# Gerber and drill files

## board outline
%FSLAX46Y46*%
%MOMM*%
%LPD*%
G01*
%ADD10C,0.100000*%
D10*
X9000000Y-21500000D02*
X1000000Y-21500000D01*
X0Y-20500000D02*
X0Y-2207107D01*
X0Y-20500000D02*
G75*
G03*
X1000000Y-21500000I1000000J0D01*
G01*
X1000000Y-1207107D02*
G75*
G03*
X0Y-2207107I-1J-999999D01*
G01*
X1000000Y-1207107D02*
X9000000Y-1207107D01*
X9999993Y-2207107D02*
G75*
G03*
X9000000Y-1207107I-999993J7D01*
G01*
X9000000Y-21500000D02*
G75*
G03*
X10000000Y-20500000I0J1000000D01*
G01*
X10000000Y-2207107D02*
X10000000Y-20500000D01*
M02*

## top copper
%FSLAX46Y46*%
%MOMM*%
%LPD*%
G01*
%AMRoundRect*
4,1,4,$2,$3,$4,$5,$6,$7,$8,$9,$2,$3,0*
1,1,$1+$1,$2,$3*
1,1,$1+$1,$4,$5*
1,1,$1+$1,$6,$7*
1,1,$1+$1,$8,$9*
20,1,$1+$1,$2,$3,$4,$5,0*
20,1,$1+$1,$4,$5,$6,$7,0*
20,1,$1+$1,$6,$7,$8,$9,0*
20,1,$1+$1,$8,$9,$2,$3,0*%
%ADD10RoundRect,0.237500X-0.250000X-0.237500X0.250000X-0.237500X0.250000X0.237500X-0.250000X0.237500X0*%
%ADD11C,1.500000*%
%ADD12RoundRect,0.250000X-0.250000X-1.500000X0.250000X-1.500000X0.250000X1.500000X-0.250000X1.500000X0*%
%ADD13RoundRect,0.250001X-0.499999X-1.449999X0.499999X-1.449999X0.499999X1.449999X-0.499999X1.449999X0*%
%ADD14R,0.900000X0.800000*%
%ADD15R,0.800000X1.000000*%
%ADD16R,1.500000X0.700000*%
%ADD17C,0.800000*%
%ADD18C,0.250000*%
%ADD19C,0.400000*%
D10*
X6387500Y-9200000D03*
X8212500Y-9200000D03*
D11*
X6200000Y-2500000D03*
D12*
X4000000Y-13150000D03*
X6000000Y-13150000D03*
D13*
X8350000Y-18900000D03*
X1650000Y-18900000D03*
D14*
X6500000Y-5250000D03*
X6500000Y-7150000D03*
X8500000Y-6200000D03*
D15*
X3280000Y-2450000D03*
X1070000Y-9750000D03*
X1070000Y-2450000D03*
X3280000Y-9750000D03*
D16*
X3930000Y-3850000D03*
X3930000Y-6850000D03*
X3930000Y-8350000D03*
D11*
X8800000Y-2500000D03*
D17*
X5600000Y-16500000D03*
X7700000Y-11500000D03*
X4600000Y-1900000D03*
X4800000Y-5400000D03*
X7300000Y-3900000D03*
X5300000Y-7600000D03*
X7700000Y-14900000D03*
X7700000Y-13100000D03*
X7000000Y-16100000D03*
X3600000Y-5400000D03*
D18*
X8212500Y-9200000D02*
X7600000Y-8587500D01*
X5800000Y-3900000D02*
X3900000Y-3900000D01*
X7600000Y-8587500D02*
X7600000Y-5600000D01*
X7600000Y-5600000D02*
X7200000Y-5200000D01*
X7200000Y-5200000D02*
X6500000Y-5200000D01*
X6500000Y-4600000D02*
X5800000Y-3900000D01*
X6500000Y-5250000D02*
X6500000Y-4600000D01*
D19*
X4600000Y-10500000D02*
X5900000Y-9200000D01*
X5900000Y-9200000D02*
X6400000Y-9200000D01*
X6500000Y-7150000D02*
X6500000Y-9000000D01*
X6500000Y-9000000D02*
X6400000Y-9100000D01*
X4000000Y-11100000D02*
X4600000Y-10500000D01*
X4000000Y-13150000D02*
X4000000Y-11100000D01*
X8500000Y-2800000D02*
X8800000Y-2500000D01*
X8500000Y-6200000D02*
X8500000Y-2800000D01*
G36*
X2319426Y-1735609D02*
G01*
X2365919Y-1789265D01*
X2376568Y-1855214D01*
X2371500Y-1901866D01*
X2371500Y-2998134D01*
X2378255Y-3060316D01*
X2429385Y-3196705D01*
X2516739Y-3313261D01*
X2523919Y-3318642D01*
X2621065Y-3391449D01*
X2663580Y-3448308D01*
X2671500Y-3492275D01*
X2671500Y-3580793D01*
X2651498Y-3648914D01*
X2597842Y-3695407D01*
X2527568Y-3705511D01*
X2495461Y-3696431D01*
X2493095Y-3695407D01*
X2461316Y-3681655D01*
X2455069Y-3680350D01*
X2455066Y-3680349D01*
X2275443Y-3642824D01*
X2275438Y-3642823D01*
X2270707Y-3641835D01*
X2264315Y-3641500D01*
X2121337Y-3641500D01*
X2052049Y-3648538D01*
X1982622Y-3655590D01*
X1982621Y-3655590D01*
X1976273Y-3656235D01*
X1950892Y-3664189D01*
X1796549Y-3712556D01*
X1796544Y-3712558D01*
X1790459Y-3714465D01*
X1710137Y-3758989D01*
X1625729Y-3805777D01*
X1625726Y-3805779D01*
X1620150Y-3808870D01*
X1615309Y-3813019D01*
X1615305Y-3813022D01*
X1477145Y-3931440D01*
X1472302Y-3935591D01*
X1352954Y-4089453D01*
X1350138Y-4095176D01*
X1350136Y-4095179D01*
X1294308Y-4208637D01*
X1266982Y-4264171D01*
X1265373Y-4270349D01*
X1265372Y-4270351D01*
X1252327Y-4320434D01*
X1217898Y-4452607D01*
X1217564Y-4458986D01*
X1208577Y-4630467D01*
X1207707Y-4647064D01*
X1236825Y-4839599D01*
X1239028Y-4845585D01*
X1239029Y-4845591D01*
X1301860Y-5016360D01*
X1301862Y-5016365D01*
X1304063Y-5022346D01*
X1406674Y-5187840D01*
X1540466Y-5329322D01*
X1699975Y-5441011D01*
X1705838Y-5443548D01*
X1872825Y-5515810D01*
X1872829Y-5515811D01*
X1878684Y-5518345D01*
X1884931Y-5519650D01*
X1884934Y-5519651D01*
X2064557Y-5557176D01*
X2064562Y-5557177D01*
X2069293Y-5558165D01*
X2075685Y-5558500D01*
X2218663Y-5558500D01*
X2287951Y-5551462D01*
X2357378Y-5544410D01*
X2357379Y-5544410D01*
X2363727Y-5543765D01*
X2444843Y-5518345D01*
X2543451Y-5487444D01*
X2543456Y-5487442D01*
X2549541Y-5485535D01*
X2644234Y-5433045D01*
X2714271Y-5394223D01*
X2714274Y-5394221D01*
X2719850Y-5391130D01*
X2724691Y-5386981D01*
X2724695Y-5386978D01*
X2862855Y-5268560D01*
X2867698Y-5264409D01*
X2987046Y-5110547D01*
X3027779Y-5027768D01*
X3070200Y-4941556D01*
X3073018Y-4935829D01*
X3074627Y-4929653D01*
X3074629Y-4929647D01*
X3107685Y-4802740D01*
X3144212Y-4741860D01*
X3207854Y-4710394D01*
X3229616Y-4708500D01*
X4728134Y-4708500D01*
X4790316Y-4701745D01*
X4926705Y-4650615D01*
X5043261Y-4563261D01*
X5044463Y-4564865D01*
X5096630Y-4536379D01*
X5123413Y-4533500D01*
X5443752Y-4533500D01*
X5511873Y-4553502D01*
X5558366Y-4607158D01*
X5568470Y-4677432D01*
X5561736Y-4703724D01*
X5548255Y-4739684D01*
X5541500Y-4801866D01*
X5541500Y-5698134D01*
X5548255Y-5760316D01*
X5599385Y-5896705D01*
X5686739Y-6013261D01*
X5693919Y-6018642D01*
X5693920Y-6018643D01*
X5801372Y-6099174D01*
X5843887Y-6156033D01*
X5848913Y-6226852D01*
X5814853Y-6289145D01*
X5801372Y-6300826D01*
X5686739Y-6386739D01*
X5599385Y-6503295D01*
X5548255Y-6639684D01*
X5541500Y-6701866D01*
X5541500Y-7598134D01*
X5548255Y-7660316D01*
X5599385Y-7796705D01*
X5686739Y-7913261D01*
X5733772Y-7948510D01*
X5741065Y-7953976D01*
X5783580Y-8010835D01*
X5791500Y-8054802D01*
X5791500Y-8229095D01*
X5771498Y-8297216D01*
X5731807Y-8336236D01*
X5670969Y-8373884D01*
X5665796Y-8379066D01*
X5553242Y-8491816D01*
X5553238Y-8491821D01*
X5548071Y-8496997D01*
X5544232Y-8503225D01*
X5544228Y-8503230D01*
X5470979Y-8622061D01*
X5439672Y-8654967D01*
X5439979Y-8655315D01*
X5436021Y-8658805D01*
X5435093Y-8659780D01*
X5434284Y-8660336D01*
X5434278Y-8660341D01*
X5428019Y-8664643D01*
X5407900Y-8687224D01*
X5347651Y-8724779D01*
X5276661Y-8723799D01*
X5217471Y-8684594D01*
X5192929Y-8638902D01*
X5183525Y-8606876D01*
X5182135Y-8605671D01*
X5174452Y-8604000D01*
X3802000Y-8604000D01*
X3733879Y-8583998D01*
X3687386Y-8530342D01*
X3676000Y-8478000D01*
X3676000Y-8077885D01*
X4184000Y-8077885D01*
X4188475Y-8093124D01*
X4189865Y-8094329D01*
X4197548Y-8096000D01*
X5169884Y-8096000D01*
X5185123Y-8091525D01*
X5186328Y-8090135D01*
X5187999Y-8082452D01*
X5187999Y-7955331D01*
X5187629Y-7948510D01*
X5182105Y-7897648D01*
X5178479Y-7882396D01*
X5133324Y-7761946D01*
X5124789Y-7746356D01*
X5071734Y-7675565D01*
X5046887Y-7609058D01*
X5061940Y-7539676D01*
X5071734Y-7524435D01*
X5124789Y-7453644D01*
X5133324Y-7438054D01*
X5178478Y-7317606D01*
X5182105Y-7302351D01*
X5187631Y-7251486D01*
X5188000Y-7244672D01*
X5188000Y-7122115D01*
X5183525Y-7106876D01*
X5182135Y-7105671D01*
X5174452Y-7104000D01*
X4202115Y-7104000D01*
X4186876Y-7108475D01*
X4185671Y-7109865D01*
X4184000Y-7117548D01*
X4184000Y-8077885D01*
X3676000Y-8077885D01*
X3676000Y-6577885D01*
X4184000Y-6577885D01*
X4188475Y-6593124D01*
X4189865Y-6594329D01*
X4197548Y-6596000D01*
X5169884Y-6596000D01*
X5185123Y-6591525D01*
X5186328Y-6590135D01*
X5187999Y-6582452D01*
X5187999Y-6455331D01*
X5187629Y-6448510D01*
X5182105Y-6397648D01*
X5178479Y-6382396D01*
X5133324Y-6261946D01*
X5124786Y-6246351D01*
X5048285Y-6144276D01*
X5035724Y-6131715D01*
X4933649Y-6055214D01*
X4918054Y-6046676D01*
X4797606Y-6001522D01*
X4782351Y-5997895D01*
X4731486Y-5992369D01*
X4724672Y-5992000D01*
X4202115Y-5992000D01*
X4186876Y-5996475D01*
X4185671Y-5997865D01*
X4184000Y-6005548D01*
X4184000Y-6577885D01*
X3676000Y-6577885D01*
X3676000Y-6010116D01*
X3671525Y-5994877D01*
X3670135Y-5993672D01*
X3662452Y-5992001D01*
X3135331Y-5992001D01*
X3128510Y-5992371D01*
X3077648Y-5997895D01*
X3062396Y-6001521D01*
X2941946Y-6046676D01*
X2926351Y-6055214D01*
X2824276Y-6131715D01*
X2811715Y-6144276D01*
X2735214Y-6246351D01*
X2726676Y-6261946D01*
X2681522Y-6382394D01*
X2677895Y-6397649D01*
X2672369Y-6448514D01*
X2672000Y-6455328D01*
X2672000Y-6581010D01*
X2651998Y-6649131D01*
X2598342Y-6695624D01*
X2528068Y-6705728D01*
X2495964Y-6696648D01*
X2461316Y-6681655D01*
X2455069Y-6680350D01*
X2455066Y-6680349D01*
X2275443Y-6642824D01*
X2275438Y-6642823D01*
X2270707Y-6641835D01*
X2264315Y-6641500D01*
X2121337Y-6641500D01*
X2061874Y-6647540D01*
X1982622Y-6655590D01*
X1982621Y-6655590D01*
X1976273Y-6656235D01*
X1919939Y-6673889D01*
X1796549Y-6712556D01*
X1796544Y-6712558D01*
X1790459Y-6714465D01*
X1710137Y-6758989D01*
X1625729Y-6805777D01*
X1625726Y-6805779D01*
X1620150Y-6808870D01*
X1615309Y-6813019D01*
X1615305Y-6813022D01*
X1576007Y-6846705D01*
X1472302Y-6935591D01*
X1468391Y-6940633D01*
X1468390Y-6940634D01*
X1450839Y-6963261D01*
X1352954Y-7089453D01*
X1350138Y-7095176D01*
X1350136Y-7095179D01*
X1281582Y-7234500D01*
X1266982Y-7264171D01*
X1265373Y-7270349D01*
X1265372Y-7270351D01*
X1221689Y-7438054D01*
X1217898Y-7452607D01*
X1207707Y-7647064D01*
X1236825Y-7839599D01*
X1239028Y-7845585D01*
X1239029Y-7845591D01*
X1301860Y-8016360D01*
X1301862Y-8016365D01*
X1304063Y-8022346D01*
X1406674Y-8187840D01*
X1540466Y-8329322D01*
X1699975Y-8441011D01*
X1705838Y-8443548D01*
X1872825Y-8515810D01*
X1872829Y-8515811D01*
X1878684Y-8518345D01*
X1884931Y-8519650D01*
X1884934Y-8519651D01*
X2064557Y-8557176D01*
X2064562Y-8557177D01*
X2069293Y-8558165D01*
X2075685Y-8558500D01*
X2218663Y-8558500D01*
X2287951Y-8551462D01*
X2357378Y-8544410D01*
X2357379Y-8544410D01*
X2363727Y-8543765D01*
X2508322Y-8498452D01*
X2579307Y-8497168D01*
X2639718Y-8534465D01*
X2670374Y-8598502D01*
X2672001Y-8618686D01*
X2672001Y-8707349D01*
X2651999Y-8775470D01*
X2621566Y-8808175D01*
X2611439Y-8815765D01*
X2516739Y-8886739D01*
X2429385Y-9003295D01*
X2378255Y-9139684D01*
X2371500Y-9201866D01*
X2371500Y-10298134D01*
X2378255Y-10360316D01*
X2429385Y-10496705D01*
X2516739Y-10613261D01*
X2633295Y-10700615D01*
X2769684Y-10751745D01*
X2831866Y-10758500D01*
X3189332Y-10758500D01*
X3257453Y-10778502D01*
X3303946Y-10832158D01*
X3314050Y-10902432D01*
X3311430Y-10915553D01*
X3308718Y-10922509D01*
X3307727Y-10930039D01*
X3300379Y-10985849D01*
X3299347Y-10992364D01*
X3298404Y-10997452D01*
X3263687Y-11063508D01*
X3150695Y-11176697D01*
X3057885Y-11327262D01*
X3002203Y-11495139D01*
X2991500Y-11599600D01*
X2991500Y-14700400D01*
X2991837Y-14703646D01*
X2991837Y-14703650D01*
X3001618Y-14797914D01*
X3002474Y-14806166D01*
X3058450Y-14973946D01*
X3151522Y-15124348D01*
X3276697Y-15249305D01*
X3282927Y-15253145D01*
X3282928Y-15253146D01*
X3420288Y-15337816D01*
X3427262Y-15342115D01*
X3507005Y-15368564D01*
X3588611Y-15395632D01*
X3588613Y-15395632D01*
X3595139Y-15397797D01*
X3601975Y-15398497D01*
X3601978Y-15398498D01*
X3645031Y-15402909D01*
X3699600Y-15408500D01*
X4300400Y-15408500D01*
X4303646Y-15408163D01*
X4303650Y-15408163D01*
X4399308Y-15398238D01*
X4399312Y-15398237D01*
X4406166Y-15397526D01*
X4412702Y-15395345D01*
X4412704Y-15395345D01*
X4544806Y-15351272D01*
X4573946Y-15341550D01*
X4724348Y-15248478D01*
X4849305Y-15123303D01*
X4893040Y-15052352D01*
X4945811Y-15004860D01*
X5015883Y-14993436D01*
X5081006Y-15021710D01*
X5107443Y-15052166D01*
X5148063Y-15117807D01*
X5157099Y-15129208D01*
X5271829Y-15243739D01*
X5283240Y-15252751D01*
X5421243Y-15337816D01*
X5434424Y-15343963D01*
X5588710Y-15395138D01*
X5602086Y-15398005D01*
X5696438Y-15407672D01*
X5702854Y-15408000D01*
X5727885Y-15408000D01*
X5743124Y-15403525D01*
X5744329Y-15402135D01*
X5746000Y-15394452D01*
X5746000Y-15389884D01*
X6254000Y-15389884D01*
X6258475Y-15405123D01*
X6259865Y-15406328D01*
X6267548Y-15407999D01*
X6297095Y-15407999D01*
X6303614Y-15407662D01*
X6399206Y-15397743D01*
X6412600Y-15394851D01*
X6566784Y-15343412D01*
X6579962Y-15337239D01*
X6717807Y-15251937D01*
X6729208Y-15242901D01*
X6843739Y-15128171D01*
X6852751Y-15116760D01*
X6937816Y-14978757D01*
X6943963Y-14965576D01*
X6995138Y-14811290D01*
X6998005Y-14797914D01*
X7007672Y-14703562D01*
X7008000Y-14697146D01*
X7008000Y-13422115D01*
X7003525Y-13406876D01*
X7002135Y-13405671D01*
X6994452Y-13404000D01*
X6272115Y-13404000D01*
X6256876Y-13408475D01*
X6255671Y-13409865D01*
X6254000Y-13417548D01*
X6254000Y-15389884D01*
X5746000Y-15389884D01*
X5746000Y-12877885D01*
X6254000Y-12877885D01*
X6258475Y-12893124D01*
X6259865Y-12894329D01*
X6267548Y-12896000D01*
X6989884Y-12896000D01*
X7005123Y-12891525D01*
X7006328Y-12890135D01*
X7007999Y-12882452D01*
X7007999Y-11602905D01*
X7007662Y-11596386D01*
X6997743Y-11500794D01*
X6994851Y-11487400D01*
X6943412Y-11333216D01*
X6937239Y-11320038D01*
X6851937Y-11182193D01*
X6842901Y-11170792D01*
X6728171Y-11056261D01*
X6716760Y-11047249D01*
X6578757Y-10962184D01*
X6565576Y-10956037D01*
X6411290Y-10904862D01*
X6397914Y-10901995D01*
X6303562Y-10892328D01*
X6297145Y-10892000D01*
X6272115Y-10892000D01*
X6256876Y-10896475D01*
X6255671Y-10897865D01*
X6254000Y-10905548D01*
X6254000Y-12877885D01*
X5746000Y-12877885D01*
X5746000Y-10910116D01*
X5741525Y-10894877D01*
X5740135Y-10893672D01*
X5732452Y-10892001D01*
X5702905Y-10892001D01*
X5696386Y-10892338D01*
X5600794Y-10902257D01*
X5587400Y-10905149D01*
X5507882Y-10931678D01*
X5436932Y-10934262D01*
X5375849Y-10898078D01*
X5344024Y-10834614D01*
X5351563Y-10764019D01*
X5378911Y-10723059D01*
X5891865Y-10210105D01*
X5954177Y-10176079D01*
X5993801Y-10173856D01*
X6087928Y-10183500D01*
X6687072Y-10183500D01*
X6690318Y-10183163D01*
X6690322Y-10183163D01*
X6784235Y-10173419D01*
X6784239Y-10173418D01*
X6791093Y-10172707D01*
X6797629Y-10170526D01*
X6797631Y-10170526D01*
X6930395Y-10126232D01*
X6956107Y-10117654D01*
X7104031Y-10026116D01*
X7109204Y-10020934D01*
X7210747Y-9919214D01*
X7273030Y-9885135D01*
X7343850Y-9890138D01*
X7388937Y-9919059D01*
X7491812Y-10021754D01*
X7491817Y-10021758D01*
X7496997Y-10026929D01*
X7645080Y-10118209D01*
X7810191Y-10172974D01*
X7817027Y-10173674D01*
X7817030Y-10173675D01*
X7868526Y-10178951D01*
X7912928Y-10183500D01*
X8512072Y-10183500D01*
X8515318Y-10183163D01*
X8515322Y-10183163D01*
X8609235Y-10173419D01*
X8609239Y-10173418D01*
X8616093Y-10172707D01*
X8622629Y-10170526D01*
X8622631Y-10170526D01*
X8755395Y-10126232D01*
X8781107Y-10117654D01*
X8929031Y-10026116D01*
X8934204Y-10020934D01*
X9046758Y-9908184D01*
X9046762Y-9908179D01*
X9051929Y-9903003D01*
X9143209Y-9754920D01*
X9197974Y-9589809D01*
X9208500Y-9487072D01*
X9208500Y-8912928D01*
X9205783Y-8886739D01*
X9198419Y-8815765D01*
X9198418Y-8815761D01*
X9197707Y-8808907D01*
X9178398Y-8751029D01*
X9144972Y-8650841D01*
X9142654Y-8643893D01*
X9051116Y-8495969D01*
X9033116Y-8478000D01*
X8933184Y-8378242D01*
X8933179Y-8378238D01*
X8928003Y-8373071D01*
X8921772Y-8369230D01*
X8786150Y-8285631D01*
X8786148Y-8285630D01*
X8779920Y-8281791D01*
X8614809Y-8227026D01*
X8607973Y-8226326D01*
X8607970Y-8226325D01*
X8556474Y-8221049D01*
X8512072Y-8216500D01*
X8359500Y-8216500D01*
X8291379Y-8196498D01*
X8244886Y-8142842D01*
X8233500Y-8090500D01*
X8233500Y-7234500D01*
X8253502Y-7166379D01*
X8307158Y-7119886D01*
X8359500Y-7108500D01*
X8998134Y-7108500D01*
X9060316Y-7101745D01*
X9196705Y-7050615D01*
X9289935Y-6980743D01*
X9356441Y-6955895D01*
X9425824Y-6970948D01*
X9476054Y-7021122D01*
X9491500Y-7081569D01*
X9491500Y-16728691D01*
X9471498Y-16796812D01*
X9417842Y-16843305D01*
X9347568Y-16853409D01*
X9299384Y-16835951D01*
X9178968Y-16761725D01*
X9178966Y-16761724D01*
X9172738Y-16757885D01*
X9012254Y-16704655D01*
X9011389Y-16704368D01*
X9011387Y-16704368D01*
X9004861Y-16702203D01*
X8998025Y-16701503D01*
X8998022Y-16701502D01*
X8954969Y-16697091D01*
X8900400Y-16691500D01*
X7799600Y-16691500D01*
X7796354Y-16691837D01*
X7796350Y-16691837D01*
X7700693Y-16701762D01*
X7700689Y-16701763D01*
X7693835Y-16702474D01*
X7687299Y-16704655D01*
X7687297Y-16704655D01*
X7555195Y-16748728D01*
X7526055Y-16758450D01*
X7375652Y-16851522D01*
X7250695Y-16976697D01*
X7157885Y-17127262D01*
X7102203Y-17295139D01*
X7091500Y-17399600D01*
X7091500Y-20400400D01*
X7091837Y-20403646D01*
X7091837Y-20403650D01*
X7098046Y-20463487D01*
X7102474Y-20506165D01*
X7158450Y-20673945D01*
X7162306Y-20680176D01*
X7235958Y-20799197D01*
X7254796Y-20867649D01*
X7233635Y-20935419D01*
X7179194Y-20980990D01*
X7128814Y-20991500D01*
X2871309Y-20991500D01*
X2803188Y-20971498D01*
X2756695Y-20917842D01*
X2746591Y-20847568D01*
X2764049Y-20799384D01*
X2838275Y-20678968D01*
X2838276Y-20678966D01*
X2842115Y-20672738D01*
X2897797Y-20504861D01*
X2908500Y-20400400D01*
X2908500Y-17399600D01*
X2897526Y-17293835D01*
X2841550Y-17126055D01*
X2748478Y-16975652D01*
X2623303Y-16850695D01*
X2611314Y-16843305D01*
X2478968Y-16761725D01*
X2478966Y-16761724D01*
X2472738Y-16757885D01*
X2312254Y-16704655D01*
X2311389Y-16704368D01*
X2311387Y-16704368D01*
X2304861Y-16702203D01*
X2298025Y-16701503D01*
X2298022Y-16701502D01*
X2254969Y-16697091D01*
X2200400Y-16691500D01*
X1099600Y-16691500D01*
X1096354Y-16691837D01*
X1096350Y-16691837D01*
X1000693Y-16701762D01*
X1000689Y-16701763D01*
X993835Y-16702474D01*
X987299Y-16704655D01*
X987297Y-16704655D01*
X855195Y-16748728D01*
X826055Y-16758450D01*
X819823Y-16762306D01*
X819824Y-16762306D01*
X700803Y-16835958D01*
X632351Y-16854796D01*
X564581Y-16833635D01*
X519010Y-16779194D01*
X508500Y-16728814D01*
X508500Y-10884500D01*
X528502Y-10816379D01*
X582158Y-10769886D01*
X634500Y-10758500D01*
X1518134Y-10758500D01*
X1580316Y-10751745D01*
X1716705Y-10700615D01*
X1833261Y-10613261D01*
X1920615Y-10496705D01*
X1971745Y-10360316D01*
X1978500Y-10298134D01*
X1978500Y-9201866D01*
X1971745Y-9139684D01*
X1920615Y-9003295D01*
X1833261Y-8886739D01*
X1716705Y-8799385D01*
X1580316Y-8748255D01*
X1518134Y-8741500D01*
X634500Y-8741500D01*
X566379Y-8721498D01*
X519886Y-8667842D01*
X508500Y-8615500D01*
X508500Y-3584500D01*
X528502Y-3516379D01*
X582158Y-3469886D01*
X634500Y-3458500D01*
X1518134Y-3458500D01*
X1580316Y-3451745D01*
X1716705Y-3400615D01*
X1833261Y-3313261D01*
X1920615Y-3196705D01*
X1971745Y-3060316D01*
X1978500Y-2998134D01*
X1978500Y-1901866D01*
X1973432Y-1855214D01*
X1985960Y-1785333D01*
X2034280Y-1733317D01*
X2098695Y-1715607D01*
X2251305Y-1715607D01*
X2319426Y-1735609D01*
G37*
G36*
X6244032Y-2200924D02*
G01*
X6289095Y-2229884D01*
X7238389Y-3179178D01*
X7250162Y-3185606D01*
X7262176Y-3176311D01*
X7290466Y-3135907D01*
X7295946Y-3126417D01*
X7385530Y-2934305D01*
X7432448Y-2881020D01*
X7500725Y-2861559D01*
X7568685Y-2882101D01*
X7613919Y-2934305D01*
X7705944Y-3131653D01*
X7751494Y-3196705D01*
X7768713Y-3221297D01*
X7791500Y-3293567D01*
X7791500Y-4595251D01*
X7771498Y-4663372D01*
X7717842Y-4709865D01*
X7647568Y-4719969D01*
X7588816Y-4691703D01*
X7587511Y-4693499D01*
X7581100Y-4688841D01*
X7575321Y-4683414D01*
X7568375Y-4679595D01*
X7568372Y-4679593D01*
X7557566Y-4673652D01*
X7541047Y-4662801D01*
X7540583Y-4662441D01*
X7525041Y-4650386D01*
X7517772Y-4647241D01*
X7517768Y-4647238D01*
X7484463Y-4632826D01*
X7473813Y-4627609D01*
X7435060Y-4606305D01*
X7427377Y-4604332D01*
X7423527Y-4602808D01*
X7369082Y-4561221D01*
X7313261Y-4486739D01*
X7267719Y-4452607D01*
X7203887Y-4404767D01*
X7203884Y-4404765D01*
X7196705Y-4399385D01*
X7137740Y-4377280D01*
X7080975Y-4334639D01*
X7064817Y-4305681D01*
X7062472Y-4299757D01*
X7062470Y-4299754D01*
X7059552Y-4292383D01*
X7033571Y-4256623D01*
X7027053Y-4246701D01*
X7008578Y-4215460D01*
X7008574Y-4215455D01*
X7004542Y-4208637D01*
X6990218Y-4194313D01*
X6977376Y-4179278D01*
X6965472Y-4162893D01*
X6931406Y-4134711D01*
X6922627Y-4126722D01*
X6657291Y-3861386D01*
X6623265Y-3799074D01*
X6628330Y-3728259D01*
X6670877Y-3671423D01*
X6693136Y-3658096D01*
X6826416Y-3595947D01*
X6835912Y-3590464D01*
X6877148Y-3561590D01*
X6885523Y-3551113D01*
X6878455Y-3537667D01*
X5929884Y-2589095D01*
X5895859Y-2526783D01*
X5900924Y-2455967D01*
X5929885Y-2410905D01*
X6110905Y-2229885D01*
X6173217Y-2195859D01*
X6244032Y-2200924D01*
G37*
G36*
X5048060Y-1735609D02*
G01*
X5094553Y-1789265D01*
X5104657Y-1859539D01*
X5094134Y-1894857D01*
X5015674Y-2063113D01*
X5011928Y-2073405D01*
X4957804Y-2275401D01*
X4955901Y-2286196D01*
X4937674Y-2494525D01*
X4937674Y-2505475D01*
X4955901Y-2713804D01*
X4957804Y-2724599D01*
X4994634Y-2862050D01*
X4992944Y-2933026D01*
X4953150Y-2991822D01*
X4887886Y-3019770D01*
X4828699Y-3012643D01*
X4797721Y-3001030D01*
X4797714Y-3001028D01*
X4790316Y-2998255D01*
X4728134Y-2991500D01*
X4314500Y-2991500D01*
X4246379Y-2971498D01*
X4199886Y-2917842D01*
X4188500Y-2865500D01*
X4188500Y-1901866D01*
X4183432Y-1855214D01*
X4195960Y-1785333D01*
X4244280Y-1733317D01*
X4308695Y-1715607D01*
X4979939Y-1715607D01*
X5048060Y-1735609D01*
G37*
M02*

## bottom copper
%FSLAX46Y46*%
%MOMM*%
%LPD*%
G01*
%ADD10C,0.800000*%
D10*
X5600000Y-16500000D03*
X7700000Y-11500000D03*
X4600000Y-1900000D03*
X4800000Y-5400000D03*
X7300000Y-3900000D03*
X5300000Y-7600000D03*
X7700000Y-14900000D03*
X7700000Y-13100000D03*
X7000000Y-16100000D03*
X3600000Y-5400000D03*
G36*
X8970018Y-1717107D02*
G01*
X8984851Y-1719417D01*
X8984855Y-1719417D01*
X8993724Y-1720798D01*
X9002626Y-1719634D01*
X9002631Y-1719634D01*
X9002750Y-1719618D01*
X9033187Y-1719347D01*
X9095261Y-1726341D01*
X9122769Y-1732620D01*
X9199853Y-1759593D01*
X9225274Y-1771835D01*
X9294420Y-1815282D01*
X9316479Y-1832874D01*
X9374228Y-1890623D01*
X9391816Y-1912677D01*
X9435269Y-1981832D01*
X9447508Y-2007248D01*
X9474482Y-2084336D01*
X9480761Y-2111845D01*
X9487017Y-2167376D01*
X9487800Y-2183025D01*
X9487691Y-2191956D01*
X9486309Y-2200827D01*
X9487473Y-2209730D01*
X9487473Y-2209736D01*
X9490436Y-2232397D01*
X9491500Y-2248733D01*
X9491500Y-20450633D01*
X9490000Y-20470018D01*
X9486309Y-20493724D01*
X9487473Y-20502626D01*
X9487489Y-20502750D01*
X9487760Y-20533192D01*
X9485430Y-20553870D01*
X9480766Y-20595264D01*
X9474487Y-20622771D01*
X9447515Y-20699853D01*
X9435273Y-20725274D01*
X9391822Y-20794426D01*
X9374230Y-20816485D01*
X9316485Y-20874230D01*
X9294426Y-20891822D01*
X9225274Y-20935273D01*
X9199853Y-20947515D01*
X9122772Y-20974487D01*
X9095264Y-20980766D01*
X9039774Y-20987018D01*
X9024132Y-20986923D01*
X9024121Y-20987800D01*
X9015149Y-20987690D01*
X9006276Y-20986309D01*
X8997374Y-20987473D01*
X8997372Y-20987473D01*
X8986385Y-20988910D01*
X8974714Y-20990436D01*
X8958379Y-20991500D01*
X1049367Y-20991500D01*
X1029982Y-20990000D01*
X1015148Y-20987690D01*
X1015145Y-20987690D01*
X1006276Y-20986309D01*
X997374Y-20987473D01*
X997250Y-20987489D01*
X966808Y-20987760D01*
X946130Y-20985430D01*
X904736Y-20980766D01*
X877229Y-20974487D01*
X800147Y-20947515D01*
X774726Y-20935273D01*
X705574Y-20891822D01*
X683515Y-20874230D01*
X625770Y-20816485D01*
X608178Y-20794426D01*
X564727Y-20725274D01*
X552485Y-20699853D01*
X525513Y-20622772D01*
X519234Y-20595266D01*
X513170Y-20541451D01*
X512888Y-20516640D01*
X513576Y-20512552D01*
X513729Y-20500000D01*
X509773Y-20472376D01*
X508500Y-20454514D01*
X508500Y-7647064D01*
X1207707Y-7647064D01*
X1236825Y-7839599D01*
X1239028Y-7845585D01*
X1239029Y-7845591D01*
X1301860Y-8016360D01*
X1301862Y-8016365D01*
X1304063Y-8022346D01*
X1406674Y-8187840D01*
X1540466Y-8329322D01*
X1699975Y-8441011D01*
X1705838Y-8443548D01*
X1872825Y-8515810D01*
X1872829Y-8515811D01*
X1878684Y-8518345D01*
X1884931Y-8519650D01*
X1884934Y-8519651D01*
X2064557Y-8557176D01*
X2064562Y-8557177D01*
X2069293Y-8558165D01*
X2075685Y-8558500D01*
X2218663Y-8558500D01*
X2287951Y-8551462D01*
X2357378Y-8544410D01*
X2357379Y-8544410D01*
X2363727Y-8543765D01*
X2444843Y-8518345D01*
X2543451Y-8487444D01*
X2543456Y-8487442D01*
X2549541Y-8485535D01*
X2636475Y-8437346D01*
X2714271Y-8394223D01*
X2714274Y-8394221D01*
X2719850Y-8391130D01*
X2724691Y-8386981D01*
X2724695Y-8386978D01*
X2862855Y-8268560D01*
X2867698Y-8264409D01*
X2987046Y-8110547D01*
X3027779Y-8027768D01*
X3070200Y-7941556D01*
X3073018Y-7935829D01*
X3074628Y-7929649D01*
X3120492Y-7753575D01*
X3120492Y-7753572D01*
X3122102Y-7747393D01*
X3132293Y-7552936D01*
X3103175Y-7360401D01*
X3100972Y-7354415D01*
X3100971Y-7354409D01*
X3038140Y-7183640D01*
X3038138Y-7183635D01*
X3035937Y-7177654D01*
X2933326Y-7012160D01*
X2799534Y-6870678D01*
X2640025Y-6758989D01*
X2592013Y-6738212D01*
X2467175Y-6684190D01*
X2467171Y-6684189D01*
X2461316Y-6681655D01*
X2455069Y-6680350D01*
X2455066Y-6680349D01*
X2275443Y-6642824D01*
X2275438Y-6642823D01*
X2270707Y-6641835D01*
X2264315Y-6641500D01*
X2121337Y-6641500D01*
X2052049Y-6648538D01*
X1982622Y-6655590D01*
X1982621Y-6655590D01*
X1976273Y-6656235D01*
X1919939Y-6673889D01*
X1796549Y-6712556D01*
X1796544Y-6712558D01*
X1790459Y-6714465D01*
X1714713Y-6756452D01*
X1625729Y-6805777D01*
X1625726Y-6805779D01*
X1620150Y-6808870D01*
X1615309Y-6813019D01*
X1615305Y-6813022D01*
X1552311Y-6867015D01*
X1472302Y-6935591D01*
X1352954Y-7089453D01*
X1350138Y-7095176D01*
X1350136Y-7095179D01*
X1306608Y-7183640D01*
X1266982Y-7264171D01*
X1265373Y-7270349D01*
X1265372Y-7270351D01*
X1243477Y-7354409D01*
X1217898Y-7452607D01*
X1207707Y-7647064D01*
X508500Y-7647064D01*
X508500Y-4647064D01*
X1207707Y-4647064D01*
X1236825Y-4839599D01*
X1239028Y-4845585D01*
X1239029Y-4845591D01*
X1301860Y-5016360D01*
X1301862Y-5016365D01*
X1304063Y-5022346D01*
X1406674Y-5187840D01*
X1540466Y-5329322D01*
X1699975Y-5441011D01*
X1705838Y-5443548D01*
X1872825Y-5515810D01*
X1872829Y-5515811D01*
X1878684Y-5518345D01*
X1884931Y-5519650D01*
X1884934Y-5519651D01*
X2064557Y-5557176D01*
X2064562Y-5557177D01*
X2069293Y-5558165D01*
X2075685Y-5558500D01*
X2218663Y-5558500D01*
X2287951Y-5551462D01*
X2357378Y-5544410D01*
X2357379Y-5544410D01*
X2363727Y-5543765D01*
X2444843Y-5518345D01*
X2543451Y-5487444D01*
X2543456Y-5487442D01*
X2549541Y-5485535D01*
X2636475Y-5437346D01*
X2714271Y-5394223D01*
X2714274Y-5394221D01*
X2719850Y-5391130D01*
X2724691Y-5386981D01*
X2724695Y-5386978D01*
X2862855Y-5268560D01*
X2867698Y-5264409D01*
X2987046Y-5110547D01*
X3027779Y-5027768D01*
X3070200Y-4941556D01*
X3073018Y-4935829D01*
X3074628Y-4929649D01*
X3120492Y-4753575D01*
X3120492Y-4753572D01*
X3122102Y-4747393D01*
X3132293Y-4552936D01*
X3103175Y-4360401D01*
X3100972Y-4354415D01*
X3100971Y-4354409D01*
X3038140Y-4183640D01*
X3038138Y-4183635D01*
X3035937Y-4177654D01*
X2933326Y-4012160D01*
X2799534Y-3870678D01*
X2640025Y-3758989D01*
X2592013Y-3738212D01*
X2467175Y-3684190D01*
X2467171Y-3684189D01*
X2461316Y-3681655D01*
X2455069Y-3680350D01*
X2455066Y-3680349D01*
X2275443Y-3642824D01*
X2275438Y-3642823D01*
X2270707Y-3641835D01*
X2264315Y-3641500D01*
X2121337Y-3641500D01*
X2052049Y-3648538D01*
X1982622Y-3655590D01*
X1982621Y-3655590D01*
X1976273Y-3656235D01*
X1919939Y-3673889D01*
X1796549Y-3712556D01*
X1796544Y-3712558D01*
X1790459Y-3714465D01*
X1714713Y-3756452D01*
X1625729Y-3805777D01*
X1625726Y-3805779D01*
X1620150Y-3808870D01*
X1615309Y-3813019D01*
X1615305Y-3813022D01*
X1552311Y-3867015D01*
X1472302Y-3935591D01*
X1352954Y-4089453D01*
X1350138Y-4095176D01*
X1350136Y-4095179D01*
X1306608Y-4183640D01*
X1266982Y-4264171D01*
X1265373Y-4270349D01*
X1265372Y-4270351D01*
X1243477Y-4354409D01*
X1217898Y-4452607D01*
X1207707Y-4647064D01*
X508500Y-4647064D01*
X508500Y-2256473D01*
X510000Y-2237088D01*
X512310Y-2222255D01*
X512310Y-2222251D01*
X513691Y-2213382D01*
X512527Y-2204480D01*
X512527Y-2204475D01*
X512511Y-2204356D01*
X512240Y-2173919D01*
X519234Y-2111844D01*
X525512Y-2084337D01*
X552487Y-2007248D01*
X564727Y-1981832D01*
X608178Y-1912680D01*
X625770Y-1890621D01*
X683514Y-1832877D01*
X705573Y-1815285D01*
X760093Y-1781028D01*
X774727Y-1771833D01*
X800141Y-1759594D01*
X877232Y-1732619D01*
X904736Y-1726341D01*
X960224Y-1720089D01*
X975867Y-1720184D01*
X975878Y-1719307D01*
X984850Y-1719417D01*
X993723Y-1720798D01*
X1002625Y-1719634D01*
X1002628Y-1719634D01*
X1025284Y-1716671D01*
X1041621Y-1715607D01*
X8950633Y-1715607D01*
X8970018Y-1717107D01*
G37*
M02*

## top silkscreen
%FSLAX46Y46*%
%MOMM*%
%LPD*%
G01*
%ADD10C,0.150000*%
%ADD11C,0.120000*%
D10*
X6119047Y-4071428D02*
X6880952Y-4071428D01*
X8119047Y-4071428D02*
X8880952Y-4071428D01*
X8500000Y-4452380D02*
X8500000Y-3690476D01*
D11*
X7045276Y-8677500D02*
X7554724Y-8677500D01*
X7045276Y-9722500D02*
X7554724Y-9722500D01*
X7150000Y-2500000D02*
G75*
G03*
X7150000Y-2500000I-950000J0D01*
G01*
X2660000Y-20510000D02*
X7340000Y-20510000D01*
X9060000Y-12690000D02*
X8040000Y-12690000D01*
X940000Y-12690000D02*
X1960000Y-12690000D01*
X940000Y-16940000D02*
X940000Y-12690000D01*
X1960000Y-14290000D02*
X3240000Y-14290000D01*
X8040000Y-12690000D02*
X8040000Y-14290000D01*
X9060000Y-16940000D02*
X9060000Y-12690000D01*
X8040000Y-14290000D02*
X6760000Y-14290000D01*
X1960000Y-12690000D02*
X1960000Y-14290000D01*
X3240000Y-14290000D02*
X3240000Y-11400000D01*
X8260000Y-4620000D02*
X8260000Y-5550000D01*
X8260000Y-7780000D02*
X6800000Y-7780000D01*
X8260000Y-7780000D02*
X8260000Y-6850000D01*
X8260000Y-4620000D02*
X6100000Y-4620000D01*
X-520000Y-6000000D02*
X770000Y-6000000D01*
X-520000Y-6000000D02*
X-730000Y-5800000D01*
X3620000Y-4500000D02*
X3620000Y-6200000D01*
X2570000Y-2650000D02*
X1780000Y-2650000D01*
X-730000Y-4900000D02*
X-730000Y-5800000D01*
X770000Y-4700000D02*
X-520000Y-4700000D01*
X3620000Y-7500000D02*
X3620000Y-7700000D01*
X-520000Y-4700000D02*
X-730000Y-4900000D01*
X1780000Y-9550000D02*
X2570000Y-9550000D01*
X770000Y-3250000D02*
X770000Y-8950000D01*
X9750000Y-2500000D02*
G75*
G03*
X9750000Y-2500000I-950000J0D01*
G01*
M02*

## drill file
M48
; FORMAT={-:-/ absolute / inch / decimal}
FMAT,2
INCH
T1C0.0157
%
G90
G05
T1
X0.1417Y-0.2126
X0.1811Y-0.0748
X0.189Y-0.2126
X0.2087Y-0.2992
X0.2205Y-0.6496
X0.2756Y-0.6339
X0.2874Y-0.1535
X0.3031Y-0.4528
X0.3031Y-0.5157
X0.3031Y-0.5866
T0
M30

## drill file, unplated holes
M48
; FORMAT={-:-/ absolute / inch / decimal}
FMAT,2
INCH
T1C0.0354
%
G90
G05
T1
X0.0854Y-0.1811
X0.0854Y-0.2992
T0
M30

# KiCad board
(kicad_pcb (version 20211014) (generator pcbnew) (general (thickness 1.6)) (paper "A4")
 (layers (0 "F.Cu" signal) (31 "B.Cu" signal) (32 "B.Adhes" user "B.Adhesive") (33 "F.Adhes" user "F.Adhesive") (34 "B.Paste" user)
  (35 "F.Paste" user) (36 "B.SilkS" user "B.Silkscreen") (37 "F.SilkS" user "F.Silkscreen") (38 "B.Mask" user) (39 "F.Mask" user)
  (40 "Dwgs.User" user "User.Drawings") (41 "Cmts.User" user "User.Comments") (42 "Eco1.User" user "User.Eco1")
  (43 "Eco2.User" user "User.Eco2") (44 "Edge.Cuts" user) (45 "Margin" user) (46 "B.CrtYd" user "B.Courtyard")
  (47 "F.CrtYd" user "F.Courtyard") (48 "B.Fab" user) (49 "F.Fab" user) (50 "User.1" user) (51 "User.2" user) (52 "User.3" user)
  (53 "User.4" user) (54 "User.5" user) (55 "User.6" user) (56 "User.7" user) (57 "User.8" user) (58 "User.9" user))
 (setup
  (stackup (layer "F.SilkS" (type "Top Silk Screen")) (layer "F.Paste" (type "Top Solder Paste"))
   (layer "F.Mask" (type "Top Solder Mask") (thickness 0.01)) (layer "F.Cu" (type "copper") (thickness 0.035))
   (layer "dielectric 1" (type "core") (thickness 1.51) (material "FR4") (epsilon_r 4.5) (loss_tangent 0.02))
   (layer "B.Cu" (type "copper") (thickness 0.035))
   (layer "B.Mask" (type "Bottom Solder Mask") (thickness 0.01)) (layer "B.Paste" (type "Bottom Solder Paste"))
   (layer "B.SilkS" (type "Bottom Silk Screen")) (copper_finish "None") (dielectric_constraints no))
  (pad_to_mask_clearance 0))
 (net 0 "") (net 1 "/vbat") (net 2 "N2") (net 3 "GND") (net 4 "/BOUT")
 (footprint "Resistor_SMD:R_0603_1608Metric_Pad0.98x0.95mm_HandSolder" (layer "F.Cu") (at 7.3 9.2)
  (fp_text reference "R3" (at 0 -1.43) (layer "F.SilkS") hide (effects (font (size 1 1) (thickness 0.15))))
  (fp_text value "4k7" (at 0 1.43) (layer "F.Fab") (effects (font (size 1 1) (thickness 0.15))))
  (fp_line (start -0.254724 -0.5225) (end 0.254724 -0.5225) (layer "F.SilkS") (width 0.12))
  (fp_line (start -0.254724 0.5225) (end 0.254724 0.5225) (layer "F.SilkS") (width 0.12))
  (pad "1" smd roundrect locked (at -0.9125 0) (size 0.975 0.95) (layers "F.Cu" "F.Paste" "F.Mask") (roundrect_rratio 0.25) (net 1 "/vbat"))
  (pad "2" smd roundrect locked (at 0.9125 0) (size 0.975 0.95) (layers "F.Cu" "F.Paste" "F.Mask") (roundrect_rratio 0.25) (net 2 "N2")))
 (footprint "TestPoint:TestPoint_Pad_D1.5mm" (layer "F.Cu") (at 6.2 2.5 180)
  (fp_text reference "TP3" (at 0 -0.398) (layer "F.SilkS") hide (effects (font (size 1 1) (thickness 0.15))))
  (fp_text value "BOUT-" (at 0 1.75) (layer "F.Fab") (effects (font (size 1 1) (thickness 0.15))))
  (fp_circle (center 0 0) (end 0 0.95) (layer "F.SilkS") (width 0.12) (fill none))
  (pad "1" smd circle locked (at 0 0 180) (size 1.5 1.5) (layers "F.Cu" "F.Mask") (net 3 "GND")))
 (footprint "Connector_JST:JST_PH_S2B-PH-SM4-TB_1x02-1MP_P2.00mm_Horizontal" (layer "F.Cu") (at 5 16)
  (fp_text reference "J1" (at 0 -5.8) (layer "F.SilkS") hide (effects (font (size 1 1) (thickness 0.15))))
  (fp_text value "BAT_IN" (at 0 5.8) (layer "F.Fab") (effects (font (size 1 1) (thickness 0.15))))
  (fp_line (start -2.34 4.51) (end 2.34 4.51) (layer "F.SilkS") (width 0.12))
  (fp_line (start 4.06 -3.31) (end 3.04 -3.31) (layer "F.SilkS") (width 0.12))
  (fp_line (start -4.06 -3.31) (end -3.04 -3.31) (layer "F.SilkS") (width 0.12))
  (fp_line (start -4.06 0.94) (end -4.06 -3.31) (layer "F.SilkS") (width 0.12))
  (fp_line (start -3.04 -1.71) (end -1.76 -1.71) (layer "F.SilkS") (width 0.12))
  (fp_line (start 3.04 -3.31) (end 3.04 -1.71) (layer "F.SilkS") (width 0.12))
  (fp_line (start 4.06 0.94) (end 4.06 -3.31) (layer "F.SilkS") (width 0.12))
  (fp_line (start 3.04 -1.71) (end 1.76 -1.71) (layer "F.SilkS") (width 0.12))
  (fp_line (start -3.04 -3.31) (end -3.04 -1.71) (layer "F.SilkS") (width 0.12))
  (fp_line (start -1.76 -1.71) (end -1.76 -4.6) (layer "F.SilkS") (width 0.12))
  (pad "1" smd roundrect locked (at -1 -2.85) (size 1 3.5) (layers "F.Cu" "F.Paste" "F.Mask") (roundrect_rratio 0.25) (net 1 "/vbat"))
  (pad "2" smd roundrect locked (at 1 -2.85) (size 1 3.5) (layers "F.Cu" "F.Paste" "F.Mask") (roundrect_rratio 0.25) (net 3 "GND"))
  (pad "MP" smd roundrect locked (at 3.35 2.9) (size 1.5 3.4) (layers "F.Cu" "F.Paste" "F.Mask") (roundrect_rratio 0.1666673333))
  (pad "MP" smd roundrect locked (at -3.35 2.9) (size 1.5 3.4) (layers "F.Cu" "F.Paste" "F.Mask") (roundrect_rratio 0.1666673333)))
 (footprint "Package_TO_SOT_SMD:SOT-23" (layer "F.Cu") (at 7.5 6.2)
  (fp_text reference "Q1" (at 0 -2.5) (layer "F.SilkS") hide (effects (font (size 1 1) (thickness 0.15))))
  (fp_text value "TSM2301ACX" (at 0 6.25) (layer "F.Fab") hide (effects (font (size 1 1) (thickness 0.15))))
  (fp_line (start 0.76 -1.58) (end 0.76 -0.65) (layer "F.SilkS") (width 0.12))
  (fp_line (start 0.76 1.58) (end -0.7 1.58) (layer "F.SilkS") (width 0.12))
  (fp_line (start 0.76 1.58) (end 0.76 0.65) (layer "F.SilkS") (width 0.12))
  (fp_line (start 0.76 -1.58) (end -1.4 -1.58) (layer "F.SilkS") (width 0.12))
  (pad "1" smd rect locked (at -1 -0.95) (size 0.9 0.8) (layers "F.Cu" "F.Paste" "F.Mask") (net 2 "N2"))
  (pad "2" smd rect locked (at -1 0.95) (size 0.9 0.8) (layers "F.Cu" "F.Paste" "F.Mask") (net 1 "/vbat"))
  (pad "3" smd rect locked (at 1 0) (size 0.9 0.8) (layers "F.Cu" "F.Paste" "F.Mask") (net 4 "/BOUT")))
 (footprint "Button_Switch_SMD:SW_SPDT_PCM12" (layer "F.Cu") (at 2.5 6.1 -90)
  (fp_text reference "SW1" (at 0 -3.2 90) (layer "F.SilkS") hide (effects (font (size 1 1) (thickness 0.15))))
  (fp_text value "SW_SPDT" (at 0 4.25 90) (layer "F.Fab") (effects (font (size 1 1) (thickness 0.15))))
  (fp_line (start -0.1 3.02) (end -0.1 1.73) (layer "F.SilkS") (width 0.12))
  (fp_line (start -0.1 3.02) (end -0.3 3.23) (layer "F.SilkS") (width 0.12))
  (fp_line (start -1.6 -1.12) (end 0.1 -1.12) (layer "F.SilkS") (width 0.12))
  (fp_line (start -3.45 -0.07) (end -3.45 0.72) (layer "F.SilkS") (width 0.12))
  (fp_line (start -1.2 3.23) (end -0.3 3.23) (layer "F.SilkS") (width 0.12))
  (fp_line (start -1.4 1.73) (end -1.4 3.02) (layer "F.SilkS") (width 0.12))
  (fp_line (start 1.4 -1.12) (end 1.6 -1.12) (layer "F.SilkS") (width 0.12))
  (fp_line (start -1.4 3.02) (end -1.2 3.23) (layer "F.SilkS") (width 0.12))
  (fp_line (start 3.45 0.72) (end 3.45 -0.07) (layer "F.SilkS") (width 0.12))
  (fp_line (start -2.85 1.73) (end 2.85 1.73) (layer "F.SilkS") (width 0.12))
  (pad "" smd rect locked (at -3.65 -0.78 270) (size 1 0.8) (layers "F.Cu" "F.Paste" "F.Mask"))
  (pad "" smd rect locked (at 3.65 1.43 270) (size 1 0.8) (layers "F.Cu" "F.Paste" "F.Mask"))
  (pad "" np_thru_hole circle locked (at -1.5 0.33 270) (size 0.9 0.9) (drill 0.9) (layers *.Cu *.Mask))
  (pad "" smd rect locked (at -3.65 1.43 270) (size 1 0.8) (layers "F.Cu" "F.Paste" "F.Mask"))
  (pad "" np_thru_hole circle locked (at 1.5 0.33 270) (size 0.9 0.9) (drill 0.9) (layers *.Cu *.Mask))
  (pad "" smd rect locked (at 3.65 -0.78 270) (size 1 0.8) (layers "F.Cu" "F.Paste" "F.Mask"))
  (pad "1" smd rect locked (at -2.25 -1.43 270) (size 0.7 1.5) (layers "F.Cu" "F.Paste" "F.Mask") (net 2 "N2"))
  (pad "2" smd rect locked (at 0.75 -1.43 270) (size 0.7 1.5) (layers "F.Cu" "F.Paste" "F.Mask") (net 3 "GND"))
  (pad "3" smd rect locked (at 2.25 -1.43 270) (size 0.7 1.5) (layers "F.Cu" "F.Paste" "F.Mask") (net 3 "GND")))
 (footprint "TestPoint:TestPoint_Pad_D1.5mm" (layer "F.Cu") (at 8.8 2.5)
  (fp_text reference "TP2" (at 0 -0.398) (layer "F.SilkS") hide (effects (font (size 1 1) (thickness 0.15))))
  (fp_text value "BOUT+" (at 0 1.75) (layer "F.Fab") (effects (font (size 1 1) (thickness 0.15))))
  (fp_circle (center 0 0) (end 0 0.95) (layer "F.SilkS") (width 0.12) (fill none))
  (pad "1" smd circle locked (at 0 0) (size 1.5 1.5) (layers "F.Cu" "F.Mask") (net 4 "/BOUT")))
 (gr_line (start 9 21.5) (end 1 21.5) (layer "Edge.Cuts") (width 0.1))
 (gr_line (start 0 20.5) (end 0 2.207107) (layer "Edge.Cuts") (width 0.1))
 (gr_arc (start 1 21.5) (mid 0.292893 21.207107) (end 0 20.5) (layer "Edge.Cuts") (width 0.1))
 (gr_arc (start 0 2.207107) (mid 0.292893 1.5) (end 1 1.207107) (layer "Edge.Cuts") (width 0.1))
 (gr_line (start 1 1.207107) (end 9 1.207107) (layer "Edge.Cuts") (width 0.1))
 (gr_arc (start 9 1.207107) (mid 9.707107 1.5) (end 10 2.207107) (layer "Edge.Cuts") (width 0.1))
 (gr_arc (start 10 20.5) (mid 9.707107 21.207107) (end 9 21.5) (layer "Edge.Cuts") (width 0.1))
 (gr_line (start 10 2.207107) (end 10 20.5) (layer "Edge.Cuts") (width 0.1))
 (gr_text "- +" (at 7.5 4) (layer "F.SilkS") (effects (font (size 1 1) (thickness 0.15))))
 (via (at 5.6 16.5) (size 0.8) (drill 0.4) (layers "F.Cu" "B.Cu") (free) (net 3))
 (via (at 7.7 11.5) (size 0.8) (drill 0.4) (layers "F.Cu" "B.Cu") (free) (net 3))
 (via (at 4.6 1.9) (size 0.8) (drill 0.4) (layers "F.Cu" "B.Cu") (free) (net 3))
 (via (at 4.8 5.4) (size 0.8) (drill 0.4) (layers "F.Cu" "B.Cu") (free) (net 3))
 (via (at 7.3 3.9) (size 0.8) (drill 0.4) (layers "F.Cu" "B.Cu") (free) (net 3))
 (via (at 5.3 7.6) (size 0.8) (drill 0.4) (layers "F.Cu" "B.Cu") (free) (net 3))
 (via (at 7.7 14.9) (size 0.8) (drill 0.4) (layers "F.Cu" "B.Cu") (free) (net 3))
 (via (at 7.7 13.1) (size 0.8) (drill 0.4) (layers "F.Cu" "B.Cu") (free) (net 3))
 (via (at 7 16.1) (size 0.8) (drill 0.4) (layers "F.Cu" "B.Cu") (free) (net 3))
 (via (at 3.6 5.4) (size 0.8) (drill 0.4) (layers "F.Cu" "B.Cu") (free) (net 3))
 (segment (start 8.2125 9.2) (end 7.6 8.5875) (width 0.25) (layer "F.Cu") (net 2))
 (segment (start 5.8 3.9) (end 3.9 3.9) (width 0.25) (layer "F.Cu") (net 2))
 (segment (start 7.6 8.5875) (end 7.6 5.6) (width 0.25) (layer "F.Cu") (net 2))
 (segment (start 7.6 5.6) (end 7.2 5.2) (width 0.25) (layer "F.Cu") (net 2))
 (segment (start 7.2 5.2) (end 6.5 5.2) (width 0.25) (layer "F.Cu") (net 2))
 (segment (start 6.5 4.6) (end 5.8 3.9) (width 0.25) (layer "F.Cu") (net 2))
 (segment (start 6.5 5.25) (end 6.5 4.6) (width 0.25) (layer "F.Cu") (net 2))
 (segment (start 4.6 10.5) (end 5.9 9.2) (width 0.4) (layer "F.Cu") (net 1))
 (segment (start 5.9 9.2) (end 6.4 9.2) (width 0.4) (layer "F.Cu") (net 1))
 (segment (start 6.5 7.15) (end 6.5 9) (width 0.4) (layer "F.Cu") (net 1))
 (segment (start 6.5 9) (end 6.4 9.1) (width 0.4) (layer "F.Cu") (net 1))
 (segment (start 4 11.1) (end 4.6 10.5) (width 0.4) (layer "F.Cu") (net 1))
 (segment (start 4 13.15) (end 4 11.1) (width 0.4) (layer "F.Cu") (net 1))
 (segment (start 8.5 2.8) (end 8.8 2.5) (width 0.4) (layer "F.Cu") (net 4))
 (segment (start 8.5 6.2) (end 8.5 2.8) (width 0.4) (layer "F.Cu") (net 4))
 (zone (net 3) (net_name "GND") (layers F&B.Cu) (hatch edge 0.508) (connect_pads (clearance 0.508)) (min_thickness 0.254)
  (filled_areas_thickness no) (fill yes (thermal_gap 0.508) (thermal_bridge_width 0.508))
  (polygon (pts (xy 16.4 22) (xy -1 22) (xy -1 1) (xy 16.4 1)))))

